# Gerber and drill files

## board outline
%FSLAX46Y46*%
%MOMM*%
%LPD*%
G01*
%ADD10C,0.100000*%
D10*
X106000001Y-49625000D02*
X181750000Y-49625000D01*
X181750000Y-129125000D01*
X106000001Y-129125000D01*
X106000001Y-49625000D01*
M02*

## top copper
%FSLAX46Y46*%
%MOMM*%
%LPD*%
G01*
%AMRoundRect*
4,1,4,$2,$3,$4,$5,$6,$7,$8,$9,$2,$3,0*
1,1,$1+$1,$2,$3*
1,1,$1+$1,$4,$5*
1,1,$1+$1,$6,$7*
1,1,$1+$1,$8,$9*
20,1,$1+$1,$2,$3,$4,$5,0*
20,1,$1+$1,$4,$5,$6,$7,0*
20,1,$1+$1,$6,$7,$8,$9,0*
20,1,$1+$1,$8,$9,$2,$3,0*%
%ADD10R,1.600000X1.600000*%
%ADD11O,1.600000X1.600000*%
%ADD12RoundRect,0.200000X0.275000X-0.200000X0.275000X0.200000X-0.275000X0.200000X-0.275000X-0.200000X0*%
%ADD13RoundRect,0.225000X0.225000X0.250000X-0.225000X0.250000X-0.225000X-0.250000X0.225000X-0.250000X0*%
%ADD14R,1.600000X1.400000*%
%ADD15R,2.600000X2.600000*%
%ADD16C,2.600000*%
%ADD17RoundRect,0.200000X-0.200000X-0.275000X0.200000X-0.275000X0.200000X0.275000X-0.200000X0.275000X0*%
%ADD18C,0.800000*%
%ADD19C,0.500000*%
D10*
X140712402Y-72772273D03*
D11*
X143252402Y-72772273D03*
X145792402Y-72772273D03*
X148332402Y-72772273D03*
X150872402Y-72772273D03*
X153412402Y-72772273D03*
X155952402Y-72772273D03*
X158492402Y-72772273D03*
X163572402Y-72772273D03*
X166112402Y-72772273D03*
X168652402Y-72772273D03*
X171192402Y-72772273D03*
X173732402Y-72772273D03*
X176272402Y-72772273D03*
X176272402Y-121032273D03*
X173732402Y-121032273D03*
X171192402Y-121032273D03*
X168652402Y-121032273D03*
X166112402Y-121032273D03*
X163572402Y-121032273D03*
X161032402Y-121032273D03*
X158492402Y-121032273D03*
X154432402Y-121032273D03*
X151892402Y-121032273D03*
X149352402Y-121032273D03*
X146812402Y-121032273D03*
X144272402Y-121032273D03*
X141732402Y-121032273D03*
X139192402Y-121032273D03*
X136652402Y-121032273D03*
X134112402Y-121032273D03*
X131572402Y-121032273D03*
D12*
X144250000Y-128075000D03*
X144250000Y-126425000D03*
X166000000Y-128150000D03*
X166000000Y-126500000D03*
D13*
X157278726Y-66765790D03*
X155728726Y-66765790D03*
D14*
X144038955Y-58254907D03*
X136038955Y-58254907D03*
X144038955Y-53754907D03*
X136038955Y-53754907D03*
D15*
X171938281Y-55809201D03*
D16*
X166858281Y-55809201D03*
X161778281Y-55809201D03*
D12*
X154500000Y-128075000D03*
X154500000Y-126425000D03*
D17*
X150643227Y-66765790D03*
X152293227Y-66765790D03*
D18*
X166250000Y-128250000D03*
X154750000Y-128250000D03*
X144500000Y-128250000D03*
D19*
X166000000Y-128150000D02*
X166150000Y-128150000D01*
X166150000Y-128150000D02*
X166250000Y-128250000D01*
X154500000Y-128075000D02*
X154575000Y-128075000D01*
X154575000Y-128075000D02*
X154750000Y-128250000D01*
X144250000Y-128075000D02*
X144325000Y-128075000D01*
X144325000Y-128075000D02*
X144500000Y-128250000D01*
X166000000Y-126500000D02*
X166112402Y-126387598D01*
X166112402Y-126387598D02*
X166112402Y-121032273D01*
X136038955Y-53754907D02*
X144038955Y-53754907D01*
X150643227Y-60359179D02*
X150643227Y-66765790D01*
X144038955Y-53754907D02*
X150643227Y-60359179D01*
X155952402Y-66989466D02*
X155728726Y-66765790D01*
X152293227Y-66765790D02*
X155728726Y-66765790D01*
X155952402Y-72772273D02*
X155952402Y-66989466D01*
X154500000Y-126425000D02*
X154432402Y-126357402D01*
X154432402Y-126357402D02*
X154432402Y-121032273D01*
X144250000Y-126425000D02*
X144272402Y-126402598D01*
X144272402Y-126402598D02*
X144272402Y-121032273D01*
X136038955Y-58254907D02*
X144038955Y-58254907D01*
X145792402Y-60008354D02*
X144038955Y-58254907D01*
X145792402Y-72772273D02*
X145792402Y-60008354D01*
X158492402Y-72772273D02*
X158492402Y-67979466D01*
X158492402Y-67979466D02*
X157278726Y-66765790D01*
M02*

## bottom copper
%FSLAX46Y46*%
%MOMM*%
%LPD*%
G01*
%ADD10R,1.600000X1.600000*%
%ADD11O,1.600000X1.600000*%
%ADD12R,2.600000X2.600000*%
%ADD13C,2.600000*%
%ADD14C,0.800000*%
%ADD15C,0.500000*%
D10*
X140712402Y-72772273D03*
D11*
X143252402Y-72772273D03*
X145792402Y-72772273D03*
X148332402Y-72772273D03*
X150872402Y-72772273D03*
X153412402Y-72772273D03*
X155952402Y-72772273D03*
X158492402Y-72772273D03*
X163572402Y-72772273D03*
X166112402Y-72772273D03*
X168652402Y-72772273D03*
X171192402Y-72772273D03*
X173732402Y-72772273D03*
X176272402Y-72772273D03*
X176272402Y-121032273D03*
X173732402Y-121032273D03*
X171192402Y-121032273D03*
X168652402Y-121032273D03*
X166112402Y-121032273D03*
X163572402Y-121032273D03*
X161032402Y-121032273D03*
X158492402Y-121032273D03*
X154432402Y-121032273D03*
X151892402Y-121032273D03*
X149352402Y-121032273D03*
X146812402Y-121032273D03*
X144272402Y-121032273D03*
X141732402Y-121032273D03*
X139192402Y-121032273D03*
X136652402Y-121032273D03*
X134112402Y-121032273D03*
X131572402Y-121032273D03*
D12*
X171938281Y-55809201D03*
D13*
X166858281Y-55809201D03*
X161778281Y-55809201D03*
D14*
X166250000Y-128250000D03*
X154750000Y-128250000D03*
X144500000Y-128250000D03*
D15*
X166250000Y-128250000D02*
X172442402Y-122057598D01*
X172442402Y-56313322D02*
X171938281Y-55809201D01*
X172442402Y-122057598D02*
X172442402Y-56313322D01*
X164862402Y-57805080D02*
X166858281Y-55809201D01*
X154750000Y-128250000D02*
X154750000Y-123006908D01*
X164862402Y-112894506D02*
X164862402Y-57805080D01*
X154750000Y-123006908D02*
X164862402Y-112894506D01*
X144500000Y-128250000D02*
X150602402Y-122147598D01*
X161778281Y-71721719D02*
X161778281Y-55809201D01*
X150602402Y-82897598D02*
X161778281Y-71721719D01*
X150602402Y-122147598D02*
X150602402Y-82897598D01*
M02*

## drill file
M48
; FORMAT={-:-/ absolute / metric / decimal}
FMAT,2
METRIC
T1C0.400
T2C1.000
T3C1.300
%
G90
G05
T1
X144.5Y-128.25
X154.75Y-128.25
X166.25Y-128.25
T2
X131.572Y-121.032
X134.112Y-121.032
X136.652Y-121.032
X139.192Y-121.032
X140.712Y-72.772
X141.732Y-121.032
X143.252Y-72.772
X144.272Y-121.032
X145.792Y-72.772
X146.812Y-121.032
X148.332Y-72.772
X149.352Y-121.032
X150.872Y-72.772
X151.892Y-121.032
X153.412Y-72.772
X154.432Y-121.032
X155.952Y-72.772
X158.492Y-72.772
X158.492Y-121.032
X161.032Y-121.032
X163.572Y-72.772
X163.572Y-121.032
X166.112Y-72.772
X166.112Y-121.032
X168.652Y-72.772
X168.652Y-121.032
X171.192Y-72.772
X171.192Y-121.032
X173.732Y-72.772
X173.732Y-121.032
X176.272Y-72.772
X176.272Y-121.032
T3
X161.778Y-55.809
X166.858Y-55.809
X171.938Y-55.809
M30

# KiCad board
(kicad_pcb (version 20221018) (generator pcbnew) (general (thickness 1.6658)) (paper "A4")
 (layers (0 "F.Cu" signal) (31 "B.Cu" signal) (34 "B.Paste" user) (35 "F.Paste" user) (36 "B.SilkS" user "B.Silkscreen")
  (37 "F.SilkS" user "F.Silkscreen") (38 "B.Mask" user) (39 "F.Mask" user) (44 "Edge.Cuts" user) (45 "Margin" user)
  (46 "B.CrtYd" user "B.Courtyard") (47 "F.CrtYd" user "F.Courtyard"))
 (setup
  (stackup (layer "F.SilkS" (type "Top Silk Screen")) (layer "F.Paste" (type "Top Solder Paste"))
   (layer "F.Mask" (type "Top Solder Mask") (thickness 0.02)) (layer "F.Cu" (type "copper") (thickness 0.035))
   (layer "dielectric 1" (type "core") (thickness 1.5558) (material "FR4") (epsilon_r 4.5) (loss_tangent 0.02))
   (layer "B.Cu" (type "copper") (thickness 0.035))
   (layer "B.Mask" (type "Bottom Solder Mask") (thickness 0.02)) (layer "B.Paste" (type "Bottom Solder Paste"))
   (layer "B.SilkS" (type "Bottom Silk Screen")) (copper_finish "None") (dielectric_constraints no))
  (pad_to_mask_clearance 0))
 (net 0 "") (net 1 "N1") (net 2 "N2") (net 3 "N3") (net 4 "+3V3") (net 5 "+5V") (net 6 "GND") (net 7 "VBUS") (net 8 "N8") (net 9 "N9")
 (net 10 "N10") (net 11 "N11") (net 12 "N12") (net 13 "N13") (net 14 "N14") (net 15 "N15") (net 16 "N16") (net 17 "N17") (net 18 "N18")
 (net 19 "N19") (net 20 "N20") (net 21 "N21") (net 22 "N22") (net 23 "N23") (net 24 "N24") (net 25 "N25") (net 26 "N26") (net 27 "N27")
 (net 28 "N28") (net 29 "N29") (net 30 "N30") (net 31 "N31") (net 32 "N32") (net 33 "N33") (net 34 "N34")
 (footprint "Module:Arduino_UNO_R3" (layer "F.Cu") (at 140.712402 72.772273)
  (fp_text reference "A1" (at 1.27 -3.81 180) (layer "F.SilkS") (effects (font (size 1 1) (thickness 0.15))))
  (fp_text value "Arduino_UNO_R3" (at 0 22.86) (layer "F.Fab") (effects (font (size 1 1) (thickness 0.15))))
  (pad "1" thru_hole rect (at 0 0 90) (size 1.6 1.6) (drill 1) (layers "*.Cu" "*.Mask") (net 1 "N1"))
  (pad "2" thru_hole oval (at 2.54 0 90) (size 1.6 1.6) (drill 1) (layers "*.Cu" "*.Mask") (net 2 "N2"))
  (pad "3" thru_hole oval (at 5.08 0 90) (size 1.6 1.6) (drill 1) (layers "*.Cu" "*.Mask") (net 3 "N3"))
  (pad "4" thru_hole oval (at 7.62 0 90) (size 1.6 1.6) (drill 1) (layers "*.Cu" "*.Mask") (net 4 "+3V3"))
  (pad "5" thru_hole oval (at 10.16 0 90) (size 1.6 1.6) (drill 1) (layers "*.Cu" "*.Mask") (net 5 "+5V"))
  (pad "6" thru_hole oval (at 12.7 0 90) (size 1.6 1.6) (drill 1) (layers "*.Cu" "*.Mask") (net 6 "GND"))
  (pad "7" thru_hole oval (at 15.24 0 90) (size 1.6 1.6) (drill 1) (layers "*.Cu" "*.Mask") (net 6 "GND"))
  (pad "8" thru_hole oval (at 17.78 0 90) (size 1.6 1.6) (drill 1) (layers "*.Cu" "*.Mask") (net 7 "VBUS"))
  (pad "9" thru_hole oval (at 22.86 0 90) (size 1.6 1.6) (drill 1) (layers "*.Cu" "*.Mask") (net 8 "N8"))
  (pad "10" thru_hole oval (at 25.4 0 90) (size 1.6 1.6) (drill 1) (layers "*.Cu" "*.Mask") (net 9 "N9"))
  (pad "11" thru_hole oval (at 27.94 0 90) (size 1.6 1.6) (drill 1) (layers "*.Cu" "*.Mask") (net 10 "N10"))
  (pad "12" thru_hole oval (at 30.48 0 90) (size 1.6 1.6) (drill 1) (layers "*.Cu" "*.Mask") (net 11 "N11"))
  (pad "13" thru_hole oval (at 33.02 0 90) (size 1.6 1.6) (drill 1) (layers "*.Cu" "*.Mask") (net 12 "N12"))
  (pad "14" thru_hole oval (at 35.56 0 90) (size 1.6 1.6) (drill 1) (layers "*.Cu" "*.Mask") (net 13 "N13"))
  (pad "15" thru_hole oval (at 35.56 48.26 90) (size 1.6 1.6) (drill 1) (layers "*.Cu" "*.Mask") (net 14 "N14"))
  (pad "16" thru_hole oval (at 33.02 48.26 90) (size 1.6 1.6) (drill 1) (layers "*.Cu" "*.Mask") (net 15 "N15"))
  (pad "17" thru_hole oval (at 30.48 48.26 90) (size 1.6 1.6) (drill 1) (layers "*.Cu" "*.Mask") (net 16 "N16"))
  (pad "18" thru_hole oval (at 27.94 48.26 90) (size 1.6 1.6) (drill 1) (layers "*.Cu" "*.Mask") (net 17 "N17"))
  (pad "19" thru_hole oval (at 25.4 48.26 90) (size 1.6 1.6) (drill 1) (layers "*.Cu" "*.Mask") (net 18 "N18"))
  (pad "20" thru_hole oval (at 22.86 48.26 90) (size 1.6 1.6) (drill 1) (layers "*.Cu" "*.Mask") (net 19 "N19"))
  (pad "21" thru_hole oval (at 20.32 48.26 90) (size 1.6 1.6) (drill 1) (layers "*.Cu" "*.Mask") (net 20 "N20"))
  (pad "22" thru_hole oval (at 17.78 48.26 90) (size 1.6 1.6) (drill 1) (layers "*.Cu" "*.Mask") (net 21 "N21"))
  (pad "23" thru_hole oval (at 13.72 48.26 90) (size 1.6 1.6) (drill 1) (layers "*.Cu" "*.Mask") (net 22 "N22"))
  (pad "24" thru_hole oval (at 11.18 48.26 90) (size 1.6 1.6) (drill 1) (layers "*.Cu" "*.Mask") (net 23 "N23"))
  (pad "25" thru_hole oval (at 8.64 48.26 90) (size 1.6 1.6) (drill 1) (layers "*.Cu" "*.Mask") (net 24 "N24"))
  (pad "26" thru_hole oval (at 6.1 48.26 90) (size 1.6 1.6) (drill 1) (layers "*.Cu" "*.Mask") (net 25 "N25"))
  (pad "27" thru_hole oval (at 3.56 48.26 90) (size 1.6 1.6) (drill 1) (layers "*.Cu" "*.Mask") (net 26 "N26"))
  (pad "28" thru_hole oval (at 1.02 48.26 90) (size 1.6 1.6) (drill 1) (layers "*.Cu" "*.Mask") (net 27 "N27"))
  (pad "29" thru_hole oval (at -1.52 48.26 90) (size 1.6 1.6) (drill 1) (layers "*.Cu" "*.Mask") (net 6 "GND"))
  (pad "30" thru_hole oval (at -4.06 48.26 90) (size 1.6 1.6) (drill 1) (layers "*.Cu" "*.Mask") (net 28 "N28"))
  (pad "31" thru_hole oval (at -6.6 48.26 90) (size 1.6 1.6) (drill 1) (layers "*.Cu" "*.Mask") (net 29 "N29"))
  (pad "32" thru_hole oval (at -9.14 48.26 90) (size 1.6 1.6) (drill 1) (layers "*.Cu" "*.Mask") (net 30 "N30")))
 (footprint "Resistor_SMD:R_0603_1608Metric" (layer "F.Cu") (at 144.25 127.25 90)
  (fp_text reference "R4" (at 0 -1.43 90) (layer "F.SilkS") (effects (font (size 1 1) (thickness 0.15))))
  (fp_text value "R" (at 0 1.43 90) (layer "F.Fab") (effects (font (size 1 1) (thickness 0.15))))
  (pad "1" smd roundrect (at -0.825 0 90) (size 0.8 0.95) (layers "F.Cu" "F.Paste" "F.Mask") (roundrect_rratio 0.25) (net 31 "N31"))
  (pad "2" smd roundrect (at 0.825 0 90) (size 0.8 0.95) (layers "F.Cu" "F.Paste" "F.Mask") (roundrect_rratio 0.25) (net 26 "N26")))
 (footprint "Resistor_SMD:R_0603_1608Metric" (layer "F.Cu") (at 166 127.325 90)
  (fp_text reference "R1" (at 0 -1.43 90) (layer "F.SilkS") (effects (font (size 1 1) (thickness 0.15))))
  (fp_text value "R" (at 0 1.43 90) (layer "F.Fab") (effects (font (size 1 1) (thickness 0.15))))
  (pad "1" smd roundrect (at -0.825 0 90) (size 0.8 0.95) (layers "F.Cu" "F.Paste" "F.Mask") (roundrect_rratio 0.25) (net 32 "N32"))
  (pad "2" smd roundrect (at 0.825 0 90) (size 0.8 0.95) (layers "F.Cu" "F.Paste" "F.Mask") (roundrect_rratio 0.25) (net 18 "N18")))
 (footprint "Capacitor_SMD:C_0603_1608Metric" (layer "F.Cu") (at 156.503726 66.76579 180)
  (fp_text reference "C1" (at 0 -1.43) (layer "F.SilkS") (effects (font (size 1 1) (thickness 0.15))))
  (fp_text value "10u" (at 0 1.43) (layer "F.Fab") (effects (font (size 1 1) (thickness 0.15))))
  (pad "1" smd roundrect (at -0.775 0 180) (size 0.9 0.95) (layers "F.Cu" "F.Paste" "F.Mask") (roundrect_rratio 0.25) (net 7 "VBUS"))
  (pad "2" smd roundrect (at 0.775 0 180) (size 0.9 0.95) (layers "F.Cu" "F.Paste" "F.Mask") (roundrect_rratio 0.25) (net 6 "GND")))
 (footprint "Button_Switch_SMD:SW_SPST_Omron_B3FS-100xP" (layer "F.Cu") (at 140.038955 56.004907 180)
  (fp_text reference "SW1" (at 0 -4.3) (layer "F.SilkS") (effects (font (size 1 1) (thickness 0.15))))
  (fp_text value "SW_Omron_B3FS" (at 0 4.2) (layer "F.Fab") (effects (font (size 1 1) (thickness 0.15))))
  (pad "1" smd rect (at -4 -2.25) (size 1.6 1.4) (layers "F.Cu" "F.Paste" "F.Mask") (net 3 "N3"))
  (pad "1" smd rect (at 4 -2.25) (size 1.6 1.4) (layers "F.Cu" "F.Paste" "F.Mask") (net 3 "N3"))
  (pad "2" smd rect (at -4 2.25) (size 1.6 1.4) (layers "F.Cu" "F.Paste" "F.Mask") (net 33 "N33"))
  (pad "2" smd rect (at 4 2.25) (size 1.6 1.4) (layers "F.Cu" "F.Paste" "F.Mask") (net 33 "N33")))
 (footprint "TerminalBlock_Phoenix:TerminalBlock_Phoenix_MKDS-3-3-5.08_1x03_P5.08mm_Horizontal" (layer "F.Cu") (at 171.938281 55.809201 180)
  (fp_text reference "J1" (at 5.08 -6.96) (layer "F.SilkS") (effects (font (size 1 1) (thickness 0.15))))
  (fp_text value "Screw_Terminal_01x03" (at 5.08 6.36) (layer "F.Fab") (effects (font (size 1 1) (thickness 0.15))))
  (pad "1" thru_hole rect (at 0 0 180) (size 2.6 2.6) (drill 1.3) (layers "*.Cu" "*.Mask") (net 32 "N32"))
  (pad "2" thru_hole circle (at 5.08 0 180) (size 2.6 2.6) (drill 1.3) (layers "*.Cu" "*.Mask") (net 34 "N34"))
  (pad "3" thru_hole circle (at 10.16 0 180) (size 2.6 2.6) (drill 1.3) (layers "*.Cu" "*.Mask") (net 31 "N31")))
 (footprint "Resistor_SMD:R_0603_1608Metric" (layer "F.Cu") (at 154.5 127.25 90)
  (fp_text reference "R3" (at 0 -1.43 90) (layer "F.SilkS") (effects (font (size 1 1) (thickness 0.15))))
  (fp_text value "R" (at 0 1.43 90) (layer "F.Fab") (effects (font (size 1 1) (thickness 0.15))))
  (pad "1" smd roundrect (at -0.825 0 90) (size 0.8 0.95) (layers "F.Cu" "F.Paste" "F.Mask") (roundrect_rratio 0.25) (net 34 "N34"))
  (pad "2" smd roundrect (at 0.825 0 90) (size 0.8 0.95) (layers "F.Cu" "F.Paste" "F.Mask") (roundrect_rratio 0.25) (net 22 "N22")))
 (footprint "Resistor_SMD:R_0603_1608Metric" (layer "F.Cu") (at 151.468227 66.76579)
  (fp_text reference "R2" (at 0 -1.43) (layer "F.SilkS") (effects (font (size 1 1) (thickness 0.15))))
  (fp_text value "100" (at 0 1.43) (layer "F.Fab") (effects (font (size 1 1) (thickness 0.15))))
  (pad "1" smd roundrect (at -0.825 0) (size 0.8 0.95) (layers "F.Cu" "F.Paste" "F.Mask") (roundrect_rratio 0.25) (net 33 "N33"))
  (pad "2" smd roundrect (at 0.825 0) (size 0.8 0.95) (layers "F.Cu" "F.Paste" "F.Mask") (roundrect_rratio 0.25) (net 6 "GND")))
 (gr_rect (start 106.000001 49.625) (end 181.75 129.125) (stroke (width 0.1) (type default)) (fill none) (layer "Edge.Cuts"))
 (segment (start 166 128.15) (end 166.15 128.15) (width 0.5) (layer "F.Cu") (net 32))
 (segment (start 166.15 128.15) (end 166.25 128.25) (width 0.5) (layer "F.Cu") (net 32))
 (via (at 166.25 128.25) (size 0.8) (drill 0.4) (layers "F.Cu" "B.Cu") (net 32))
 (segment (start 166.25 128.25) (end 172.442402 122.057598) (width 0.5) (layer "B.Cu") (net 32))
 (segment (start 172.442402 56.313322) (end 171.938281 55.809201) (width 0.5) (layer "B.Cu") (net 32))
 (segment (start 172.442402 122.057598) (end 172.442402 56.313322) (width 0.5) (layer "B.Cu") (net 32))
 (segment (start 154.5 128.075) (end 154.575 128.075) (width 0.5) (layer "F.Cu") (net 34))
 (segment (start 154.575 128.075) (end 154.75 128.25) (width 0.5) (layer "F.Cu") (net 34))
 (via (at 154.75 128.25) (size 0.8) (drill 0.4) (layers "F.Cu" "B.Cu") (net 34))
 (segment (start 164.862402 57.80508) (end 166.858281 55.809201) (width 0.5) (layer "B.Cu") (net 34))
 (segment (start 154.75 128.25) (end 154.75 123.006908) (width 0.5) (layer "B.Cu") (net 34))
 (segment (start 164.862402 112.894506) (end 164.862402 57.80508) (width 0.5) (layer "B.Cu") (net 34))
 (segment (start 154.75 123.006908) (end 164.862402 112.894506) (width 0.5) (layer "B.Cu") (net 34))
 (segment (start 144.25 128.075) (end 144.325 128.075) (width 0.5) (layer "F.Cu") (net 31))
 (segment (start 144.325 128.075) (end 144.5 128.25) (width 0.5) (layer "F.Cu") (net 31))
 (via (at 144.5 128.25) (size 0.8) (drill 0.4) (layers "F.Cu" "B.Cu") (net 31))
 (segment (start 144.5 128.25) (end 150.602402 122.147598) (width 0.5) (layer "B.Cu") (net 31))
 (segment (start 161.778281 71.721719) (end 161.778281 55.809201) (width 0.5) (layer "B.Cu") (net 31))
 (segment (start 150.602402 82.897598) (end 161.778281 71.721719) (width 0.5) (layer "B.Cu") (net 31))
 (segment (start 150.602402 122.147598) (end 150.602402 82.897598) (width 0.5) (layer "B.Cu") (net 31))
 (segment (start 166 126.5) (end 166.112402 126.387598) (width 0.5) (layer "F.Cu") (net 18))
 (segment (start 166.112402 126.387598) (end 166.112402 121.032273) (width 0.5) (layer "F.Cu") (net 18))
 (segment (start 136.038955 53.754907) (end 144.038955 53.754907) (width 0.5) (layer "F.Cu") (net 33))
 (segment (start 150.643227 60.359179) (end 150.643227 66.76579) (width 0.5) (layer "F.Cu") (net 33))
 (segment (start 144.038955 53.754907) (end 150.643227 60.359179) (width 0.5) (layer "F.Cu") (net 33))
 (segment (start 155.952402 66.989466) (end 155.728726 66.76579) (width 0.5) (layer "F.Cu") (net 6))
 (segment (start 152.293227 66.76579) (end 155.728726 66.76579) (width 0.5) (layer "F.Cu") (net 6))
 (segment (start 155.952402 72.772273) (end 155.952402 66.989466) (width 0.5) (layer "F.Cu") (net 6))
 (segment (start 154.5 126.425) (end 154.432402 126.357402) (width 0.5) (layer "F.Cu") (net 22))
 (segment (start 154.432402 126.357402) (end 154.432402 121.032273) (width 0.5) (layer "F.Cu") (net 22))
 (segment (start 144.25 126.425) (end 144.272402 126.402598) (width 0.5) (layer "F.Cu") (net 26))
 (segment (start 144.272402 126.402598) (end 144.272402 121.032273) (width 0.5) (layer "F.Cu") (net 26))
 (segment (start 136.038955 58.254907) (end 144.038955 58.254907) (width 0.5) (layer "F.Cu") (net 3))
 (segment (start 145.792402 60.008354) (end 144.038955 58.254907) (width 0.5) (layer "F.Cu") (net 3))
 (segment (start 145.792402 72.772273) (end 145.792402 60.008354) (width 0.5) (layer "F.Cu") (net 3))
 (segment (start 158.492402 72.772273) (end 158.492402 67.979466) (width 0.5) (layer "F.Cu") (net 7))
 (segment (start 158.492402 67.979466) (end 157.278726 66.76579) (width 0.5) (layer "F.Cu") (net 7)))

